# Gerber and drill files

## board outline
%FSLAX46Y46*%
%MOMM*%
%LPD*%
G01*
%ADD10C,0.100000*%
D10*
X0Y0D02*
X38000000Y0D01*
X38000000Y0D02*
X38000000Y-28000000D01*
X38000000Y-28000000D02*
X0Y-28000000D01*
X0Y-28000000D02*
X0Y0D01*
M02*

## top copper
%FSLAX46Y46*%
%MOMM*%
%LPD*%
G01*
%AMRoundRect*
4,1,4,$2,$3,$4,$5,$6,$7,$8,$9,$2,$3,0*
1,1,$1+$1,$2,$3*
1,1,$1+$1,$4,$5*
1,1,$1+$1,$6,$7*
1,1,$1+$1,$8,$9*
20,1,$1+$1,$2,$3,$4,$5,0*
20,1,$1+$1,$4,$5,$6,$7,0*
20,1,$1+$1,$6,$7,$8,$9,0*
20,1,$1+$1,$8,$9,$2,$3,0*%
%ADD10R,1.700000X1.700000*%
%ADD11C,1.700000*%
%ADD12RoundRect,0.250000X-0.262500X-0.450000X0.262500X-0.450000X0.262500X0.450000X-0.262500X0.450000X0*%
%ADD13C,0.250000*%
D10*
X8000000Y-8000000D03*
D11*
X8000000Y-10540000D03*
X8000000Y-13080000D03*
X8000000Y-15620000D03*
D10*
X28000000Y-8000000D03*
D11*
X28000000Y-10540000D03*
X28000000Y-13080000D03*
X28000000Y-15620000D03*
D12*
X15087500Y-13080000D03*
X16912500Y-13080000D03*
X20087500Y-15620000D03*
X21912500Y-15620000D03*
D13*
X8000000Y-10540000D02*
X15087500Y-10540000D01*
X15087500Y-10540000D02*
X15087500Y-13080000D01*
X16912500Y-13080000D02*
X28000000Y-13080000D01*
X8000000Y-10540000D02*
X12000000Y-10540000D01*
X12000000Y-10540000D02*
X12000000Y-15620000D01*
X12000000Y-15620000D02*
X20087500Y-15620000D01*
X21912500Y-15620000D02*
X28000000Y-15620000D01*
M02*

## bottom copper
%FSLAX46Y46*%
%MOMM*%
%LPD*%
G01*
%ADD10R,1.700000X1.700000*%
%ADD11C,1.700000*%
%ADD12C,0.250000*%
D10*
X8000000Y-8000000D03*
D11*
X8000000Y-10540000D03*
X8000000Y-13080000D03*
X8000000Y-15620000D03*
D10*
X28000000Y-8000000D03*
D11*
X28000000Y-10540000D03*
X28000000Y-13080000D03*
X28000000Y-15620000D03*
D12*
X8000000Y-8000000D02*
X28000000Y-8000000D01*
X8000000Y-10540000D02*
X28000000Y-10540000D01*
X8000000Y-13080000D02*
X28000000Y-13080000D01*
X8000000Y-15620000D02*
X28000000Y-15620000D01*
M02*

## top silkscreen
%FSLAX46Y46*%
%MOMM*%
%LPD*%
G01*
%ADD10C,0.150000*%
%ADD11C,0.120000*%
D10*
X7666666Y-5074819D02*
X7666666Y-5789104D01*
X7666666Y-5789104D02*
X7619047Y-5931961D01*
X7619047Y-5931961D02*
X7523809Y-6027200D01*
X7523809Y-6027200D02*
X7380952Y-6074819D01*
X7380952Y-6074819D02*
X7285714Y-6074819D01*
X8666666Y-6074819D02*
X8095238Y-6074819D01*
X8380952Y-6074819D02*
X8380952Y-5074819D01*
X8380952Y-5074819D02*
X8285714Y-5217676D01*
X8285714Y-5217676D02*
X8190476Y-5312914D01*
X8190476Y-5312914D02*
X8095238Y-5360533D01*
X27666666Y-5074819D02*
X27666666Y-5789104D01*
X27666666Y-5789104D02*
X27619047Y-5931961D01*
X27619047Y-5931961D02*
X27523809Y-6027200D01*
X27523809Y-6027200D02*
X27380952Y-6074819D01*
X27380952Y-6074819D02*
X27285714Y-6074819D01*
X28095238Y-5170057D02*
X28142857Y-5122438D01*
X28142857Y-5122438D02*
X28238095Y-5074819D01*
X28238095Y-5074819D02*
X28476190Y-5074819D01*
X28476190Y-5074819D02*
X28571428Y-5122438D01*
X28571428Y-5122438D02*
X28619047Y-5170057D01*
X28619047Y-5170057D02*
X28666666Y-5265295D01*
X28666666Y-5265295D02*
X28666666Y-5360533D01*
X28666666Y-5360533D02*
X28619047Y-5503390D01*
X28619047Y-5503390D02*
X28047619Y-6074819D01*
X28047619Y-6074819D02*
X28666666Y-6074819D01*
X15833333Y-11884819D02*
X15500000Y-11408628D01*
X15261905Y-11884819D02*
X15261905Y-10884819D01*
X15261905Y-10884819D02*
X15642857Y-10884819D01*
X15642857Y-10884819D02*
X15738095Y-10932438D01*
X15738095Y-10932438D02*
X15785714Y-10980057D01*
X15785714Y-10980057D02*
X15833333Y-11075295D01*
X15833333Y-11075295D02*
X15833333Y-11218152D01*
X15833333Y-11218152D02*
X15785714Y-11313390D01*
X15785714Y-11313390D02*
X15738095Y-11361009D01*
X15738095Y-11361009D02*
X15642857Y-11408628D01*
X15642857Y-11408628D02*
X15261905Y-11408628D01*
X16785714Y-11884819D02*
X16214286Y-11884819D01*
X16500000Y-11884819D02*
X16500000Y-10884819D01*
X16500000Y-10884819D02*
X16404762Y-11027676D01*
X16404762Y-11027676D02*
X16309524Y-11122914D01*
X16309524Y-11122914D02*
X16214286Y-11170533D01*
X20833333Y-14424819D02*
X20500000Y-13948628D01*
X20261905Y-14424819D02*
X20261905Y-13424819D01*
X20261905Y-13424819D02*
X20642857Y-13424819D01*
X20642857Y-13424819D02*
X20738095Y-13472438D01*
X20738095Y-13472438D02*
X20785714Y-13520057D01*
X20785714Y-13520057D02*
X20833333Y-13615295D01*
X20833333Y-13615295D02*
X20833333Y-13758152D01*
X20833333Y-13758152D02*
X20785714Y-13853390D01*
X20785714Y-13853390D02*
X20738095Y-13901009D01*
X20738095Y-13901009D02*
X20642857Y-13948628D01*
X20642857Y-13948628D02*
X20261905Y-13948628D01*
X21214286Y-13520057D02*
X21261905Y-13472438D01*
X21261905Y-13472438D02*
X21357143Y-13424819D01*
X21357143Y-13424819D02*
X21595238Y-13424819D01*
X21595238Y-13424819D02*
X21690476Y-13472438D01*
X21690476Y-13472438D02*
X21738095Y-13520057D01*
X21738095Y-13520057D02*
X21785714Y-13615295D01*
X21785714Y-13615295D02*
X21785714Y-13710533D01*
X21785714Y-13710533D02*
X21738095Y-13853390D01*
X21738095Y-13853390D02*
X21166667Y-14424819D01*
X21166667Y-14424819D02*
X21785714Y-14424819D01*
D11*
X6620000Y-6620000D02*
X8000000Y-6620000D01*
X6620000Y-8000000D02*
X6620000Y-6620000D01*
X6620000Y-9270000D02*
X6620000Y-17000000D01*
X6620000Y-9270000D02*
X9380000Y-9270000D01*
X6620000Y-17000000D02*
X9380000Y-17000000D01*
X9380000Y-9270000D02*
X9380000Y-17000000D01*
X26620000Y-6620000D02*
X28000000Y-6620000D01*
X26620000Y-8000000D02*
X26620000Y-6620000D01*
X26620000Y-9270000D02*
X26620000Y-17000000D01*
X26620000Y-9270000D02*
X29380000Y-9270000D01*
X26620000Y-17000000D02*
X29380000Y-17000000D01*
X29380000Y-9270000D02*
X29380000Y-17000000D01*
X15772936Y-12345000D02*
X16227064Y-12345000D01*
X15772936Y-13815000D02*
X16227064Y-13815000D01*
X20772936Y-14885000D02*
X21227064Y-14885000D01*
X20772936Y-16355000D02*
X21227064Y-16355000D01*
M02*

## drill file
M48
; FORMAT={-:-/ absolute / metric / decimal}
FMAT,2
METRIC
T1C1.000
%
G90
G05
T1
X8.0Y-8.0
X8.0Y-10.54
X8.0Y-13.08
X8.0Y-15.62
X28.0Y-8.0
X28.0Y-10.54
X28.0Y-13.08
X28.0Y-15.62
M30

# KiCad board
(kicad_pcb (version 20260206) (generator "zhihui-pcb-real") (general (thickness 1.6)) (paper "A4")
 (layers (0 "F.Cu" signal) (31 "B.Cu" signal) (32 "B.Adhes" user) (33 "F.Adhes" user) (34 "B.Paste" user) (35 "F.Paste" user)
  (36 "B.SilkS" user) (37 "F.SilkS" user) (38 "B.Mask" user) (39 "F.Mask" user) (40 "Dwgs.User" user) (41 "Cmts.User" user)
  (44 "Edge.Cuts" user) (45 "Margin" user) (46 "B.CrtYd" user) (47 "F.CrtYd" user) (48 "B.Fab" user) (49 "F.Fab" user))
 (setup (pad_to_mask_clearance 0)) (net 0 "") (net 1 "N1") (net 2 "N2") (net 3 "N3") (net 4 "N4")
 (gr_line (start 0 0) (end 38 0) (stroke (width 0.1) (type default)) (layer "Edge.Cuts"))
 (gr_line (start 38 0) (end 38 28) (stroke (width 0.1) (type default)) (layer "Edge.Cuts"))
 (gr_line (start 38 28) (end 0 28) (stroke (width 0.1) (type default)) (layer "Edge.Cuts"))
 (gr_line (start 0 28) (end 0 0) (stroke (width 0.1) (type default)) (layer "Edge.Cuts"))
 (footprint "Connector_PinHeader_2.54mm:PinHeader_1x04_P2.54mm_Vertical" (layer "F.Cu")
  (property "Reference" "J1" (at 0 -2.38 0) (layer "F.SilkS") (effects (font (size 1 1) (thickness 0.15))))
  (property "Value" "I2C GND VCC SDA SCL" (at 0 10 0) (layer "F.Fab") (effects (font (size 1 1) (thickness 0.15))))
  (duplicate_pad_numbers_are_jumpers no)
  (fp_line (start -1.38 -1.38) (end 0 -1.38) (stroke (width 0.12) (type solid)) (layer "F.SilkS"))
  (fp_line (start -1.38 0) (end -1.38 -1.38) (stroke (width 0.12) (type solid)) (layer "F.SilkS"))
  (fp_line (start -1.38 1.27) (end -1.38 9) (stroke (width 0.12) (type solid)) (layer "F.SilkS"))
  (fp_line (start -1.38 1.27) (end 1.38 1.27) (stroke (width 0.12) (type solid)) (layer "F.SilkS"))
  (fp_line (start -1.38 9) (end 1.38 9) (stroke (width 0.12) (type solid)) (layer "F.SilkS"))
  (fp_line (start 1.38 1.27) (end 1.38 9) (stroke (width 0.12) (type solid)) (layer "F.SilkS"))
  (pad "1" thru_hole rect (at 0 0) (size 1.7 1.7) (drill 1) (layers "*.Cu" "*.Mask") (remove_unused_layers no) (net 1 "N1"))
  (pad "2" thru_hole circle (at 0 2.54) (size 1.7 1.7) (drill 1) (layers "*.Cu" "*.Mask") (remove_unused_layers no) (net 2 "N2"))
  (pad "3" thru_hole circle (at 0 5.08) (size 1.7 1.7) (drill 1) (layers "*.Cu" "*.Mask") (remove_unused_layers no) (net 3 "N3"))
  (pad "4" thru_hole circle (at 0 7.62) (size 1.7 1.7) (drill 1) (layers "*.Cu" "*.Mask") (remove_unused_layers no) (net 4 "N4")) (at 8 8 0))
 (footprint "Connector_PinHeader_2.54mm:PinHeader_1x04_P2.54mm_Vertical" (layer "F.Cu")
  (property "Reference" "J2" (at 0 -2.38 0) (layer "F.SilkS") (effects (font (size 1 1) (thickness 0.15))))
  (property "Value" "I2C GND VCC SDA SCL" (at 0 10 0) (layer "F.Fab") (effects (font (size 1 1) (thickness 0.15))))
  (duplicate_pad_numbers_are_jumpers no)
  (fp_line (start -1.38 -1.38) (end 0 -1.38) (stroke (width 0.12) (type solid)) (layer "F.SilkS"))
  (fp_line (start -1.38 0) (end -1.38 -1.38) (stroke (width 0.12) (type solid)) (layer "F.SilkS"))
  (fp_line (start -1.38 1.27) (end -1.38 9) (stroke (width 0.12) (type solid)) (layer "F.SilkS"))
  (fp_line (start -1.38 1.27) (end 1.38 1.27) (stroke (width 0.12) (type solid)) (layer "F.SilkS"))
  (fp_line (start -1.38 9) (end 1.38 9) (stroke (width 0.12) (type solid)) (layer "F.SilkS"))
  (fp_line (start 1.38 1.27) (end 1.38 9) (stroke (width 0.12) (type solid)) (layer "F.SilkS"))
  (pad "1" thru_hole rect (at 0 0) (size 1.7 1.7) (drill 1) (layers "*.Cu" "*.Mask") (remove_unused_layers no) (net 1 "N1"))
  (pad "2" thru_hole circle (at 0 2.54) (size 1.7 1.7) (drill 1) (layers "*.Cu" "*.Mask") (remove_unused_layers no) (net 2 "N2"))
  (pad "3" thru_hole circle (at 0 5.08) (size 1.7 1.7) (drill 1) (layers "*.Cu" "*.Mask") (remove_unused_layers no) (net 3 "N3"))
  (pad "4" thru_hole circle (at 0 7.62) (size 1.7 1.7) (drill 1) (layers "*.Cu" "*.Mask") (remove_unused_layers no) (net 4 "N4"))
  (at 28 8 0))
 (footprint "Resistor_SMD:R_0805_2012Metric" (layer "F.Cu")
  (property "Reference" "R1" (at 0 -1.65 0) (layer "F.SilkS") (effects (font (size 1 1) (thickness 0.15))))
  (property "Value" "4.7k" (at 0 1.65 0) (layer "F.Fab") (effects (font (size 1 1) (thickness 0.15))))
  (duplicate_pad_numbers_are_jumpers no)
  (fp_line (start -0.227064 -0.735) (end 0.227064 -0.735) (stroke (width 0.12) (type solid)) (layer "F.SilkS"))
  (fp_line (start -0.227064 0.735) (end 0.227064 0.735) (stroke (width 0.12) (type solid)) (layer "F.SilkS"))
  (pad "1" smd roundrect (at -0.9125 0) (size 1.025 1.4) (layers "F.Cu" "F.Mask" "F.Paste") (roundrect_rratio 0.243902) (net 2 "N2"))
  (pad "2" smd roundrect (at 0.9125 0) (size 1.025 1.4) (layers "F.Cu" "F.Mask" "F.Paste") (roundrect_rratio 0.243902) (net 3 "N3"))
  (at 16 13.08 0))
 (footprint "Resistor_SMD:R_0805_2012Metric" (layer "F.Cu")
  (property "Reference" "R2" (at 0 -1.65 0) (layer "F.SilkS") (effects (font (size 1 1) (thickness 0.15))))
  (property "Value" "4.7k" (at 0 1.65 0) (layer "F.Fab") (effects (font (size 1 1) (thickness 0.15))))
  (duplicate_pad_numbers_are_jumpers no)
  (fp_line (start -0.227064 -0.735) (end 0.227064 -0.735) (stroke (width 0.12) (type solid)) (layer "F.SilkS"))
  (fp_line (start -0.227064 0.735) (end 0.227064 0.735) (stroke (width 0.12) (type solid)) (layer "F.SilkS"))
  (pad "1" smd roundrect (at -0.9125 0) (size 1.025 1.4) (layers "F.Cu" "F.Mask" "F.Paste") (roundrect_rratio 0.243902) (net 2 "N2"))
  (pad "2" smd roundrect (at 0.9125 0) (size 1.025 1.4) (layers "F.Cu" "F.Mask" "F.Paste") (roundrect_rratio 0.243902) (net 4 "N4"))
  (at 21 15.62 0))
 (segment (start 8 8) (end 28 8) (width 0.25) (layer "B.Cu") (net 1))
 (segment (start 8 10.54) (end 28 10.54) (width 0.25) (layer "B.Cu") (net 2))
 (segment (start 8 13.08) (end 28 13.08) (width 0.25) (layer "B.Cu") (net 3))
 (segment (start 8 15.62) (end 28 15.62) (width 0.25) (layer "B.Cu") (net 4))
 (segment (start 8 10.54) (end 15.0875 10.54) (width 0.25) (layer "F.Cu") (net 2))
 (segment (start 15.0875 10.54) (end 15.0875 13.08) (width 0.25) (layer "F.Cu") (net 2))
 (segment (start 16.9125 13.08) (end 28 13.08) (width 0.25) (layer "F.Cu") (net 3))
 (segment (start 8 10.54) (end 12 10.54) (width 0.25) (layer "F.Cu") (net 2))
 (segment (start 12 10.54) (end 12 15.62) (width 0.25) (layer "F.Cu") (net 2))
 (segment (start 12 15.62) (end 20.0875 15.62) (width 0.25) (layer "F.Cu") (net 2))
 (segment (start 21.9125 15.62) (end 28 15.62) (width 0.25) (layer "F.Cu") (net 4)))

